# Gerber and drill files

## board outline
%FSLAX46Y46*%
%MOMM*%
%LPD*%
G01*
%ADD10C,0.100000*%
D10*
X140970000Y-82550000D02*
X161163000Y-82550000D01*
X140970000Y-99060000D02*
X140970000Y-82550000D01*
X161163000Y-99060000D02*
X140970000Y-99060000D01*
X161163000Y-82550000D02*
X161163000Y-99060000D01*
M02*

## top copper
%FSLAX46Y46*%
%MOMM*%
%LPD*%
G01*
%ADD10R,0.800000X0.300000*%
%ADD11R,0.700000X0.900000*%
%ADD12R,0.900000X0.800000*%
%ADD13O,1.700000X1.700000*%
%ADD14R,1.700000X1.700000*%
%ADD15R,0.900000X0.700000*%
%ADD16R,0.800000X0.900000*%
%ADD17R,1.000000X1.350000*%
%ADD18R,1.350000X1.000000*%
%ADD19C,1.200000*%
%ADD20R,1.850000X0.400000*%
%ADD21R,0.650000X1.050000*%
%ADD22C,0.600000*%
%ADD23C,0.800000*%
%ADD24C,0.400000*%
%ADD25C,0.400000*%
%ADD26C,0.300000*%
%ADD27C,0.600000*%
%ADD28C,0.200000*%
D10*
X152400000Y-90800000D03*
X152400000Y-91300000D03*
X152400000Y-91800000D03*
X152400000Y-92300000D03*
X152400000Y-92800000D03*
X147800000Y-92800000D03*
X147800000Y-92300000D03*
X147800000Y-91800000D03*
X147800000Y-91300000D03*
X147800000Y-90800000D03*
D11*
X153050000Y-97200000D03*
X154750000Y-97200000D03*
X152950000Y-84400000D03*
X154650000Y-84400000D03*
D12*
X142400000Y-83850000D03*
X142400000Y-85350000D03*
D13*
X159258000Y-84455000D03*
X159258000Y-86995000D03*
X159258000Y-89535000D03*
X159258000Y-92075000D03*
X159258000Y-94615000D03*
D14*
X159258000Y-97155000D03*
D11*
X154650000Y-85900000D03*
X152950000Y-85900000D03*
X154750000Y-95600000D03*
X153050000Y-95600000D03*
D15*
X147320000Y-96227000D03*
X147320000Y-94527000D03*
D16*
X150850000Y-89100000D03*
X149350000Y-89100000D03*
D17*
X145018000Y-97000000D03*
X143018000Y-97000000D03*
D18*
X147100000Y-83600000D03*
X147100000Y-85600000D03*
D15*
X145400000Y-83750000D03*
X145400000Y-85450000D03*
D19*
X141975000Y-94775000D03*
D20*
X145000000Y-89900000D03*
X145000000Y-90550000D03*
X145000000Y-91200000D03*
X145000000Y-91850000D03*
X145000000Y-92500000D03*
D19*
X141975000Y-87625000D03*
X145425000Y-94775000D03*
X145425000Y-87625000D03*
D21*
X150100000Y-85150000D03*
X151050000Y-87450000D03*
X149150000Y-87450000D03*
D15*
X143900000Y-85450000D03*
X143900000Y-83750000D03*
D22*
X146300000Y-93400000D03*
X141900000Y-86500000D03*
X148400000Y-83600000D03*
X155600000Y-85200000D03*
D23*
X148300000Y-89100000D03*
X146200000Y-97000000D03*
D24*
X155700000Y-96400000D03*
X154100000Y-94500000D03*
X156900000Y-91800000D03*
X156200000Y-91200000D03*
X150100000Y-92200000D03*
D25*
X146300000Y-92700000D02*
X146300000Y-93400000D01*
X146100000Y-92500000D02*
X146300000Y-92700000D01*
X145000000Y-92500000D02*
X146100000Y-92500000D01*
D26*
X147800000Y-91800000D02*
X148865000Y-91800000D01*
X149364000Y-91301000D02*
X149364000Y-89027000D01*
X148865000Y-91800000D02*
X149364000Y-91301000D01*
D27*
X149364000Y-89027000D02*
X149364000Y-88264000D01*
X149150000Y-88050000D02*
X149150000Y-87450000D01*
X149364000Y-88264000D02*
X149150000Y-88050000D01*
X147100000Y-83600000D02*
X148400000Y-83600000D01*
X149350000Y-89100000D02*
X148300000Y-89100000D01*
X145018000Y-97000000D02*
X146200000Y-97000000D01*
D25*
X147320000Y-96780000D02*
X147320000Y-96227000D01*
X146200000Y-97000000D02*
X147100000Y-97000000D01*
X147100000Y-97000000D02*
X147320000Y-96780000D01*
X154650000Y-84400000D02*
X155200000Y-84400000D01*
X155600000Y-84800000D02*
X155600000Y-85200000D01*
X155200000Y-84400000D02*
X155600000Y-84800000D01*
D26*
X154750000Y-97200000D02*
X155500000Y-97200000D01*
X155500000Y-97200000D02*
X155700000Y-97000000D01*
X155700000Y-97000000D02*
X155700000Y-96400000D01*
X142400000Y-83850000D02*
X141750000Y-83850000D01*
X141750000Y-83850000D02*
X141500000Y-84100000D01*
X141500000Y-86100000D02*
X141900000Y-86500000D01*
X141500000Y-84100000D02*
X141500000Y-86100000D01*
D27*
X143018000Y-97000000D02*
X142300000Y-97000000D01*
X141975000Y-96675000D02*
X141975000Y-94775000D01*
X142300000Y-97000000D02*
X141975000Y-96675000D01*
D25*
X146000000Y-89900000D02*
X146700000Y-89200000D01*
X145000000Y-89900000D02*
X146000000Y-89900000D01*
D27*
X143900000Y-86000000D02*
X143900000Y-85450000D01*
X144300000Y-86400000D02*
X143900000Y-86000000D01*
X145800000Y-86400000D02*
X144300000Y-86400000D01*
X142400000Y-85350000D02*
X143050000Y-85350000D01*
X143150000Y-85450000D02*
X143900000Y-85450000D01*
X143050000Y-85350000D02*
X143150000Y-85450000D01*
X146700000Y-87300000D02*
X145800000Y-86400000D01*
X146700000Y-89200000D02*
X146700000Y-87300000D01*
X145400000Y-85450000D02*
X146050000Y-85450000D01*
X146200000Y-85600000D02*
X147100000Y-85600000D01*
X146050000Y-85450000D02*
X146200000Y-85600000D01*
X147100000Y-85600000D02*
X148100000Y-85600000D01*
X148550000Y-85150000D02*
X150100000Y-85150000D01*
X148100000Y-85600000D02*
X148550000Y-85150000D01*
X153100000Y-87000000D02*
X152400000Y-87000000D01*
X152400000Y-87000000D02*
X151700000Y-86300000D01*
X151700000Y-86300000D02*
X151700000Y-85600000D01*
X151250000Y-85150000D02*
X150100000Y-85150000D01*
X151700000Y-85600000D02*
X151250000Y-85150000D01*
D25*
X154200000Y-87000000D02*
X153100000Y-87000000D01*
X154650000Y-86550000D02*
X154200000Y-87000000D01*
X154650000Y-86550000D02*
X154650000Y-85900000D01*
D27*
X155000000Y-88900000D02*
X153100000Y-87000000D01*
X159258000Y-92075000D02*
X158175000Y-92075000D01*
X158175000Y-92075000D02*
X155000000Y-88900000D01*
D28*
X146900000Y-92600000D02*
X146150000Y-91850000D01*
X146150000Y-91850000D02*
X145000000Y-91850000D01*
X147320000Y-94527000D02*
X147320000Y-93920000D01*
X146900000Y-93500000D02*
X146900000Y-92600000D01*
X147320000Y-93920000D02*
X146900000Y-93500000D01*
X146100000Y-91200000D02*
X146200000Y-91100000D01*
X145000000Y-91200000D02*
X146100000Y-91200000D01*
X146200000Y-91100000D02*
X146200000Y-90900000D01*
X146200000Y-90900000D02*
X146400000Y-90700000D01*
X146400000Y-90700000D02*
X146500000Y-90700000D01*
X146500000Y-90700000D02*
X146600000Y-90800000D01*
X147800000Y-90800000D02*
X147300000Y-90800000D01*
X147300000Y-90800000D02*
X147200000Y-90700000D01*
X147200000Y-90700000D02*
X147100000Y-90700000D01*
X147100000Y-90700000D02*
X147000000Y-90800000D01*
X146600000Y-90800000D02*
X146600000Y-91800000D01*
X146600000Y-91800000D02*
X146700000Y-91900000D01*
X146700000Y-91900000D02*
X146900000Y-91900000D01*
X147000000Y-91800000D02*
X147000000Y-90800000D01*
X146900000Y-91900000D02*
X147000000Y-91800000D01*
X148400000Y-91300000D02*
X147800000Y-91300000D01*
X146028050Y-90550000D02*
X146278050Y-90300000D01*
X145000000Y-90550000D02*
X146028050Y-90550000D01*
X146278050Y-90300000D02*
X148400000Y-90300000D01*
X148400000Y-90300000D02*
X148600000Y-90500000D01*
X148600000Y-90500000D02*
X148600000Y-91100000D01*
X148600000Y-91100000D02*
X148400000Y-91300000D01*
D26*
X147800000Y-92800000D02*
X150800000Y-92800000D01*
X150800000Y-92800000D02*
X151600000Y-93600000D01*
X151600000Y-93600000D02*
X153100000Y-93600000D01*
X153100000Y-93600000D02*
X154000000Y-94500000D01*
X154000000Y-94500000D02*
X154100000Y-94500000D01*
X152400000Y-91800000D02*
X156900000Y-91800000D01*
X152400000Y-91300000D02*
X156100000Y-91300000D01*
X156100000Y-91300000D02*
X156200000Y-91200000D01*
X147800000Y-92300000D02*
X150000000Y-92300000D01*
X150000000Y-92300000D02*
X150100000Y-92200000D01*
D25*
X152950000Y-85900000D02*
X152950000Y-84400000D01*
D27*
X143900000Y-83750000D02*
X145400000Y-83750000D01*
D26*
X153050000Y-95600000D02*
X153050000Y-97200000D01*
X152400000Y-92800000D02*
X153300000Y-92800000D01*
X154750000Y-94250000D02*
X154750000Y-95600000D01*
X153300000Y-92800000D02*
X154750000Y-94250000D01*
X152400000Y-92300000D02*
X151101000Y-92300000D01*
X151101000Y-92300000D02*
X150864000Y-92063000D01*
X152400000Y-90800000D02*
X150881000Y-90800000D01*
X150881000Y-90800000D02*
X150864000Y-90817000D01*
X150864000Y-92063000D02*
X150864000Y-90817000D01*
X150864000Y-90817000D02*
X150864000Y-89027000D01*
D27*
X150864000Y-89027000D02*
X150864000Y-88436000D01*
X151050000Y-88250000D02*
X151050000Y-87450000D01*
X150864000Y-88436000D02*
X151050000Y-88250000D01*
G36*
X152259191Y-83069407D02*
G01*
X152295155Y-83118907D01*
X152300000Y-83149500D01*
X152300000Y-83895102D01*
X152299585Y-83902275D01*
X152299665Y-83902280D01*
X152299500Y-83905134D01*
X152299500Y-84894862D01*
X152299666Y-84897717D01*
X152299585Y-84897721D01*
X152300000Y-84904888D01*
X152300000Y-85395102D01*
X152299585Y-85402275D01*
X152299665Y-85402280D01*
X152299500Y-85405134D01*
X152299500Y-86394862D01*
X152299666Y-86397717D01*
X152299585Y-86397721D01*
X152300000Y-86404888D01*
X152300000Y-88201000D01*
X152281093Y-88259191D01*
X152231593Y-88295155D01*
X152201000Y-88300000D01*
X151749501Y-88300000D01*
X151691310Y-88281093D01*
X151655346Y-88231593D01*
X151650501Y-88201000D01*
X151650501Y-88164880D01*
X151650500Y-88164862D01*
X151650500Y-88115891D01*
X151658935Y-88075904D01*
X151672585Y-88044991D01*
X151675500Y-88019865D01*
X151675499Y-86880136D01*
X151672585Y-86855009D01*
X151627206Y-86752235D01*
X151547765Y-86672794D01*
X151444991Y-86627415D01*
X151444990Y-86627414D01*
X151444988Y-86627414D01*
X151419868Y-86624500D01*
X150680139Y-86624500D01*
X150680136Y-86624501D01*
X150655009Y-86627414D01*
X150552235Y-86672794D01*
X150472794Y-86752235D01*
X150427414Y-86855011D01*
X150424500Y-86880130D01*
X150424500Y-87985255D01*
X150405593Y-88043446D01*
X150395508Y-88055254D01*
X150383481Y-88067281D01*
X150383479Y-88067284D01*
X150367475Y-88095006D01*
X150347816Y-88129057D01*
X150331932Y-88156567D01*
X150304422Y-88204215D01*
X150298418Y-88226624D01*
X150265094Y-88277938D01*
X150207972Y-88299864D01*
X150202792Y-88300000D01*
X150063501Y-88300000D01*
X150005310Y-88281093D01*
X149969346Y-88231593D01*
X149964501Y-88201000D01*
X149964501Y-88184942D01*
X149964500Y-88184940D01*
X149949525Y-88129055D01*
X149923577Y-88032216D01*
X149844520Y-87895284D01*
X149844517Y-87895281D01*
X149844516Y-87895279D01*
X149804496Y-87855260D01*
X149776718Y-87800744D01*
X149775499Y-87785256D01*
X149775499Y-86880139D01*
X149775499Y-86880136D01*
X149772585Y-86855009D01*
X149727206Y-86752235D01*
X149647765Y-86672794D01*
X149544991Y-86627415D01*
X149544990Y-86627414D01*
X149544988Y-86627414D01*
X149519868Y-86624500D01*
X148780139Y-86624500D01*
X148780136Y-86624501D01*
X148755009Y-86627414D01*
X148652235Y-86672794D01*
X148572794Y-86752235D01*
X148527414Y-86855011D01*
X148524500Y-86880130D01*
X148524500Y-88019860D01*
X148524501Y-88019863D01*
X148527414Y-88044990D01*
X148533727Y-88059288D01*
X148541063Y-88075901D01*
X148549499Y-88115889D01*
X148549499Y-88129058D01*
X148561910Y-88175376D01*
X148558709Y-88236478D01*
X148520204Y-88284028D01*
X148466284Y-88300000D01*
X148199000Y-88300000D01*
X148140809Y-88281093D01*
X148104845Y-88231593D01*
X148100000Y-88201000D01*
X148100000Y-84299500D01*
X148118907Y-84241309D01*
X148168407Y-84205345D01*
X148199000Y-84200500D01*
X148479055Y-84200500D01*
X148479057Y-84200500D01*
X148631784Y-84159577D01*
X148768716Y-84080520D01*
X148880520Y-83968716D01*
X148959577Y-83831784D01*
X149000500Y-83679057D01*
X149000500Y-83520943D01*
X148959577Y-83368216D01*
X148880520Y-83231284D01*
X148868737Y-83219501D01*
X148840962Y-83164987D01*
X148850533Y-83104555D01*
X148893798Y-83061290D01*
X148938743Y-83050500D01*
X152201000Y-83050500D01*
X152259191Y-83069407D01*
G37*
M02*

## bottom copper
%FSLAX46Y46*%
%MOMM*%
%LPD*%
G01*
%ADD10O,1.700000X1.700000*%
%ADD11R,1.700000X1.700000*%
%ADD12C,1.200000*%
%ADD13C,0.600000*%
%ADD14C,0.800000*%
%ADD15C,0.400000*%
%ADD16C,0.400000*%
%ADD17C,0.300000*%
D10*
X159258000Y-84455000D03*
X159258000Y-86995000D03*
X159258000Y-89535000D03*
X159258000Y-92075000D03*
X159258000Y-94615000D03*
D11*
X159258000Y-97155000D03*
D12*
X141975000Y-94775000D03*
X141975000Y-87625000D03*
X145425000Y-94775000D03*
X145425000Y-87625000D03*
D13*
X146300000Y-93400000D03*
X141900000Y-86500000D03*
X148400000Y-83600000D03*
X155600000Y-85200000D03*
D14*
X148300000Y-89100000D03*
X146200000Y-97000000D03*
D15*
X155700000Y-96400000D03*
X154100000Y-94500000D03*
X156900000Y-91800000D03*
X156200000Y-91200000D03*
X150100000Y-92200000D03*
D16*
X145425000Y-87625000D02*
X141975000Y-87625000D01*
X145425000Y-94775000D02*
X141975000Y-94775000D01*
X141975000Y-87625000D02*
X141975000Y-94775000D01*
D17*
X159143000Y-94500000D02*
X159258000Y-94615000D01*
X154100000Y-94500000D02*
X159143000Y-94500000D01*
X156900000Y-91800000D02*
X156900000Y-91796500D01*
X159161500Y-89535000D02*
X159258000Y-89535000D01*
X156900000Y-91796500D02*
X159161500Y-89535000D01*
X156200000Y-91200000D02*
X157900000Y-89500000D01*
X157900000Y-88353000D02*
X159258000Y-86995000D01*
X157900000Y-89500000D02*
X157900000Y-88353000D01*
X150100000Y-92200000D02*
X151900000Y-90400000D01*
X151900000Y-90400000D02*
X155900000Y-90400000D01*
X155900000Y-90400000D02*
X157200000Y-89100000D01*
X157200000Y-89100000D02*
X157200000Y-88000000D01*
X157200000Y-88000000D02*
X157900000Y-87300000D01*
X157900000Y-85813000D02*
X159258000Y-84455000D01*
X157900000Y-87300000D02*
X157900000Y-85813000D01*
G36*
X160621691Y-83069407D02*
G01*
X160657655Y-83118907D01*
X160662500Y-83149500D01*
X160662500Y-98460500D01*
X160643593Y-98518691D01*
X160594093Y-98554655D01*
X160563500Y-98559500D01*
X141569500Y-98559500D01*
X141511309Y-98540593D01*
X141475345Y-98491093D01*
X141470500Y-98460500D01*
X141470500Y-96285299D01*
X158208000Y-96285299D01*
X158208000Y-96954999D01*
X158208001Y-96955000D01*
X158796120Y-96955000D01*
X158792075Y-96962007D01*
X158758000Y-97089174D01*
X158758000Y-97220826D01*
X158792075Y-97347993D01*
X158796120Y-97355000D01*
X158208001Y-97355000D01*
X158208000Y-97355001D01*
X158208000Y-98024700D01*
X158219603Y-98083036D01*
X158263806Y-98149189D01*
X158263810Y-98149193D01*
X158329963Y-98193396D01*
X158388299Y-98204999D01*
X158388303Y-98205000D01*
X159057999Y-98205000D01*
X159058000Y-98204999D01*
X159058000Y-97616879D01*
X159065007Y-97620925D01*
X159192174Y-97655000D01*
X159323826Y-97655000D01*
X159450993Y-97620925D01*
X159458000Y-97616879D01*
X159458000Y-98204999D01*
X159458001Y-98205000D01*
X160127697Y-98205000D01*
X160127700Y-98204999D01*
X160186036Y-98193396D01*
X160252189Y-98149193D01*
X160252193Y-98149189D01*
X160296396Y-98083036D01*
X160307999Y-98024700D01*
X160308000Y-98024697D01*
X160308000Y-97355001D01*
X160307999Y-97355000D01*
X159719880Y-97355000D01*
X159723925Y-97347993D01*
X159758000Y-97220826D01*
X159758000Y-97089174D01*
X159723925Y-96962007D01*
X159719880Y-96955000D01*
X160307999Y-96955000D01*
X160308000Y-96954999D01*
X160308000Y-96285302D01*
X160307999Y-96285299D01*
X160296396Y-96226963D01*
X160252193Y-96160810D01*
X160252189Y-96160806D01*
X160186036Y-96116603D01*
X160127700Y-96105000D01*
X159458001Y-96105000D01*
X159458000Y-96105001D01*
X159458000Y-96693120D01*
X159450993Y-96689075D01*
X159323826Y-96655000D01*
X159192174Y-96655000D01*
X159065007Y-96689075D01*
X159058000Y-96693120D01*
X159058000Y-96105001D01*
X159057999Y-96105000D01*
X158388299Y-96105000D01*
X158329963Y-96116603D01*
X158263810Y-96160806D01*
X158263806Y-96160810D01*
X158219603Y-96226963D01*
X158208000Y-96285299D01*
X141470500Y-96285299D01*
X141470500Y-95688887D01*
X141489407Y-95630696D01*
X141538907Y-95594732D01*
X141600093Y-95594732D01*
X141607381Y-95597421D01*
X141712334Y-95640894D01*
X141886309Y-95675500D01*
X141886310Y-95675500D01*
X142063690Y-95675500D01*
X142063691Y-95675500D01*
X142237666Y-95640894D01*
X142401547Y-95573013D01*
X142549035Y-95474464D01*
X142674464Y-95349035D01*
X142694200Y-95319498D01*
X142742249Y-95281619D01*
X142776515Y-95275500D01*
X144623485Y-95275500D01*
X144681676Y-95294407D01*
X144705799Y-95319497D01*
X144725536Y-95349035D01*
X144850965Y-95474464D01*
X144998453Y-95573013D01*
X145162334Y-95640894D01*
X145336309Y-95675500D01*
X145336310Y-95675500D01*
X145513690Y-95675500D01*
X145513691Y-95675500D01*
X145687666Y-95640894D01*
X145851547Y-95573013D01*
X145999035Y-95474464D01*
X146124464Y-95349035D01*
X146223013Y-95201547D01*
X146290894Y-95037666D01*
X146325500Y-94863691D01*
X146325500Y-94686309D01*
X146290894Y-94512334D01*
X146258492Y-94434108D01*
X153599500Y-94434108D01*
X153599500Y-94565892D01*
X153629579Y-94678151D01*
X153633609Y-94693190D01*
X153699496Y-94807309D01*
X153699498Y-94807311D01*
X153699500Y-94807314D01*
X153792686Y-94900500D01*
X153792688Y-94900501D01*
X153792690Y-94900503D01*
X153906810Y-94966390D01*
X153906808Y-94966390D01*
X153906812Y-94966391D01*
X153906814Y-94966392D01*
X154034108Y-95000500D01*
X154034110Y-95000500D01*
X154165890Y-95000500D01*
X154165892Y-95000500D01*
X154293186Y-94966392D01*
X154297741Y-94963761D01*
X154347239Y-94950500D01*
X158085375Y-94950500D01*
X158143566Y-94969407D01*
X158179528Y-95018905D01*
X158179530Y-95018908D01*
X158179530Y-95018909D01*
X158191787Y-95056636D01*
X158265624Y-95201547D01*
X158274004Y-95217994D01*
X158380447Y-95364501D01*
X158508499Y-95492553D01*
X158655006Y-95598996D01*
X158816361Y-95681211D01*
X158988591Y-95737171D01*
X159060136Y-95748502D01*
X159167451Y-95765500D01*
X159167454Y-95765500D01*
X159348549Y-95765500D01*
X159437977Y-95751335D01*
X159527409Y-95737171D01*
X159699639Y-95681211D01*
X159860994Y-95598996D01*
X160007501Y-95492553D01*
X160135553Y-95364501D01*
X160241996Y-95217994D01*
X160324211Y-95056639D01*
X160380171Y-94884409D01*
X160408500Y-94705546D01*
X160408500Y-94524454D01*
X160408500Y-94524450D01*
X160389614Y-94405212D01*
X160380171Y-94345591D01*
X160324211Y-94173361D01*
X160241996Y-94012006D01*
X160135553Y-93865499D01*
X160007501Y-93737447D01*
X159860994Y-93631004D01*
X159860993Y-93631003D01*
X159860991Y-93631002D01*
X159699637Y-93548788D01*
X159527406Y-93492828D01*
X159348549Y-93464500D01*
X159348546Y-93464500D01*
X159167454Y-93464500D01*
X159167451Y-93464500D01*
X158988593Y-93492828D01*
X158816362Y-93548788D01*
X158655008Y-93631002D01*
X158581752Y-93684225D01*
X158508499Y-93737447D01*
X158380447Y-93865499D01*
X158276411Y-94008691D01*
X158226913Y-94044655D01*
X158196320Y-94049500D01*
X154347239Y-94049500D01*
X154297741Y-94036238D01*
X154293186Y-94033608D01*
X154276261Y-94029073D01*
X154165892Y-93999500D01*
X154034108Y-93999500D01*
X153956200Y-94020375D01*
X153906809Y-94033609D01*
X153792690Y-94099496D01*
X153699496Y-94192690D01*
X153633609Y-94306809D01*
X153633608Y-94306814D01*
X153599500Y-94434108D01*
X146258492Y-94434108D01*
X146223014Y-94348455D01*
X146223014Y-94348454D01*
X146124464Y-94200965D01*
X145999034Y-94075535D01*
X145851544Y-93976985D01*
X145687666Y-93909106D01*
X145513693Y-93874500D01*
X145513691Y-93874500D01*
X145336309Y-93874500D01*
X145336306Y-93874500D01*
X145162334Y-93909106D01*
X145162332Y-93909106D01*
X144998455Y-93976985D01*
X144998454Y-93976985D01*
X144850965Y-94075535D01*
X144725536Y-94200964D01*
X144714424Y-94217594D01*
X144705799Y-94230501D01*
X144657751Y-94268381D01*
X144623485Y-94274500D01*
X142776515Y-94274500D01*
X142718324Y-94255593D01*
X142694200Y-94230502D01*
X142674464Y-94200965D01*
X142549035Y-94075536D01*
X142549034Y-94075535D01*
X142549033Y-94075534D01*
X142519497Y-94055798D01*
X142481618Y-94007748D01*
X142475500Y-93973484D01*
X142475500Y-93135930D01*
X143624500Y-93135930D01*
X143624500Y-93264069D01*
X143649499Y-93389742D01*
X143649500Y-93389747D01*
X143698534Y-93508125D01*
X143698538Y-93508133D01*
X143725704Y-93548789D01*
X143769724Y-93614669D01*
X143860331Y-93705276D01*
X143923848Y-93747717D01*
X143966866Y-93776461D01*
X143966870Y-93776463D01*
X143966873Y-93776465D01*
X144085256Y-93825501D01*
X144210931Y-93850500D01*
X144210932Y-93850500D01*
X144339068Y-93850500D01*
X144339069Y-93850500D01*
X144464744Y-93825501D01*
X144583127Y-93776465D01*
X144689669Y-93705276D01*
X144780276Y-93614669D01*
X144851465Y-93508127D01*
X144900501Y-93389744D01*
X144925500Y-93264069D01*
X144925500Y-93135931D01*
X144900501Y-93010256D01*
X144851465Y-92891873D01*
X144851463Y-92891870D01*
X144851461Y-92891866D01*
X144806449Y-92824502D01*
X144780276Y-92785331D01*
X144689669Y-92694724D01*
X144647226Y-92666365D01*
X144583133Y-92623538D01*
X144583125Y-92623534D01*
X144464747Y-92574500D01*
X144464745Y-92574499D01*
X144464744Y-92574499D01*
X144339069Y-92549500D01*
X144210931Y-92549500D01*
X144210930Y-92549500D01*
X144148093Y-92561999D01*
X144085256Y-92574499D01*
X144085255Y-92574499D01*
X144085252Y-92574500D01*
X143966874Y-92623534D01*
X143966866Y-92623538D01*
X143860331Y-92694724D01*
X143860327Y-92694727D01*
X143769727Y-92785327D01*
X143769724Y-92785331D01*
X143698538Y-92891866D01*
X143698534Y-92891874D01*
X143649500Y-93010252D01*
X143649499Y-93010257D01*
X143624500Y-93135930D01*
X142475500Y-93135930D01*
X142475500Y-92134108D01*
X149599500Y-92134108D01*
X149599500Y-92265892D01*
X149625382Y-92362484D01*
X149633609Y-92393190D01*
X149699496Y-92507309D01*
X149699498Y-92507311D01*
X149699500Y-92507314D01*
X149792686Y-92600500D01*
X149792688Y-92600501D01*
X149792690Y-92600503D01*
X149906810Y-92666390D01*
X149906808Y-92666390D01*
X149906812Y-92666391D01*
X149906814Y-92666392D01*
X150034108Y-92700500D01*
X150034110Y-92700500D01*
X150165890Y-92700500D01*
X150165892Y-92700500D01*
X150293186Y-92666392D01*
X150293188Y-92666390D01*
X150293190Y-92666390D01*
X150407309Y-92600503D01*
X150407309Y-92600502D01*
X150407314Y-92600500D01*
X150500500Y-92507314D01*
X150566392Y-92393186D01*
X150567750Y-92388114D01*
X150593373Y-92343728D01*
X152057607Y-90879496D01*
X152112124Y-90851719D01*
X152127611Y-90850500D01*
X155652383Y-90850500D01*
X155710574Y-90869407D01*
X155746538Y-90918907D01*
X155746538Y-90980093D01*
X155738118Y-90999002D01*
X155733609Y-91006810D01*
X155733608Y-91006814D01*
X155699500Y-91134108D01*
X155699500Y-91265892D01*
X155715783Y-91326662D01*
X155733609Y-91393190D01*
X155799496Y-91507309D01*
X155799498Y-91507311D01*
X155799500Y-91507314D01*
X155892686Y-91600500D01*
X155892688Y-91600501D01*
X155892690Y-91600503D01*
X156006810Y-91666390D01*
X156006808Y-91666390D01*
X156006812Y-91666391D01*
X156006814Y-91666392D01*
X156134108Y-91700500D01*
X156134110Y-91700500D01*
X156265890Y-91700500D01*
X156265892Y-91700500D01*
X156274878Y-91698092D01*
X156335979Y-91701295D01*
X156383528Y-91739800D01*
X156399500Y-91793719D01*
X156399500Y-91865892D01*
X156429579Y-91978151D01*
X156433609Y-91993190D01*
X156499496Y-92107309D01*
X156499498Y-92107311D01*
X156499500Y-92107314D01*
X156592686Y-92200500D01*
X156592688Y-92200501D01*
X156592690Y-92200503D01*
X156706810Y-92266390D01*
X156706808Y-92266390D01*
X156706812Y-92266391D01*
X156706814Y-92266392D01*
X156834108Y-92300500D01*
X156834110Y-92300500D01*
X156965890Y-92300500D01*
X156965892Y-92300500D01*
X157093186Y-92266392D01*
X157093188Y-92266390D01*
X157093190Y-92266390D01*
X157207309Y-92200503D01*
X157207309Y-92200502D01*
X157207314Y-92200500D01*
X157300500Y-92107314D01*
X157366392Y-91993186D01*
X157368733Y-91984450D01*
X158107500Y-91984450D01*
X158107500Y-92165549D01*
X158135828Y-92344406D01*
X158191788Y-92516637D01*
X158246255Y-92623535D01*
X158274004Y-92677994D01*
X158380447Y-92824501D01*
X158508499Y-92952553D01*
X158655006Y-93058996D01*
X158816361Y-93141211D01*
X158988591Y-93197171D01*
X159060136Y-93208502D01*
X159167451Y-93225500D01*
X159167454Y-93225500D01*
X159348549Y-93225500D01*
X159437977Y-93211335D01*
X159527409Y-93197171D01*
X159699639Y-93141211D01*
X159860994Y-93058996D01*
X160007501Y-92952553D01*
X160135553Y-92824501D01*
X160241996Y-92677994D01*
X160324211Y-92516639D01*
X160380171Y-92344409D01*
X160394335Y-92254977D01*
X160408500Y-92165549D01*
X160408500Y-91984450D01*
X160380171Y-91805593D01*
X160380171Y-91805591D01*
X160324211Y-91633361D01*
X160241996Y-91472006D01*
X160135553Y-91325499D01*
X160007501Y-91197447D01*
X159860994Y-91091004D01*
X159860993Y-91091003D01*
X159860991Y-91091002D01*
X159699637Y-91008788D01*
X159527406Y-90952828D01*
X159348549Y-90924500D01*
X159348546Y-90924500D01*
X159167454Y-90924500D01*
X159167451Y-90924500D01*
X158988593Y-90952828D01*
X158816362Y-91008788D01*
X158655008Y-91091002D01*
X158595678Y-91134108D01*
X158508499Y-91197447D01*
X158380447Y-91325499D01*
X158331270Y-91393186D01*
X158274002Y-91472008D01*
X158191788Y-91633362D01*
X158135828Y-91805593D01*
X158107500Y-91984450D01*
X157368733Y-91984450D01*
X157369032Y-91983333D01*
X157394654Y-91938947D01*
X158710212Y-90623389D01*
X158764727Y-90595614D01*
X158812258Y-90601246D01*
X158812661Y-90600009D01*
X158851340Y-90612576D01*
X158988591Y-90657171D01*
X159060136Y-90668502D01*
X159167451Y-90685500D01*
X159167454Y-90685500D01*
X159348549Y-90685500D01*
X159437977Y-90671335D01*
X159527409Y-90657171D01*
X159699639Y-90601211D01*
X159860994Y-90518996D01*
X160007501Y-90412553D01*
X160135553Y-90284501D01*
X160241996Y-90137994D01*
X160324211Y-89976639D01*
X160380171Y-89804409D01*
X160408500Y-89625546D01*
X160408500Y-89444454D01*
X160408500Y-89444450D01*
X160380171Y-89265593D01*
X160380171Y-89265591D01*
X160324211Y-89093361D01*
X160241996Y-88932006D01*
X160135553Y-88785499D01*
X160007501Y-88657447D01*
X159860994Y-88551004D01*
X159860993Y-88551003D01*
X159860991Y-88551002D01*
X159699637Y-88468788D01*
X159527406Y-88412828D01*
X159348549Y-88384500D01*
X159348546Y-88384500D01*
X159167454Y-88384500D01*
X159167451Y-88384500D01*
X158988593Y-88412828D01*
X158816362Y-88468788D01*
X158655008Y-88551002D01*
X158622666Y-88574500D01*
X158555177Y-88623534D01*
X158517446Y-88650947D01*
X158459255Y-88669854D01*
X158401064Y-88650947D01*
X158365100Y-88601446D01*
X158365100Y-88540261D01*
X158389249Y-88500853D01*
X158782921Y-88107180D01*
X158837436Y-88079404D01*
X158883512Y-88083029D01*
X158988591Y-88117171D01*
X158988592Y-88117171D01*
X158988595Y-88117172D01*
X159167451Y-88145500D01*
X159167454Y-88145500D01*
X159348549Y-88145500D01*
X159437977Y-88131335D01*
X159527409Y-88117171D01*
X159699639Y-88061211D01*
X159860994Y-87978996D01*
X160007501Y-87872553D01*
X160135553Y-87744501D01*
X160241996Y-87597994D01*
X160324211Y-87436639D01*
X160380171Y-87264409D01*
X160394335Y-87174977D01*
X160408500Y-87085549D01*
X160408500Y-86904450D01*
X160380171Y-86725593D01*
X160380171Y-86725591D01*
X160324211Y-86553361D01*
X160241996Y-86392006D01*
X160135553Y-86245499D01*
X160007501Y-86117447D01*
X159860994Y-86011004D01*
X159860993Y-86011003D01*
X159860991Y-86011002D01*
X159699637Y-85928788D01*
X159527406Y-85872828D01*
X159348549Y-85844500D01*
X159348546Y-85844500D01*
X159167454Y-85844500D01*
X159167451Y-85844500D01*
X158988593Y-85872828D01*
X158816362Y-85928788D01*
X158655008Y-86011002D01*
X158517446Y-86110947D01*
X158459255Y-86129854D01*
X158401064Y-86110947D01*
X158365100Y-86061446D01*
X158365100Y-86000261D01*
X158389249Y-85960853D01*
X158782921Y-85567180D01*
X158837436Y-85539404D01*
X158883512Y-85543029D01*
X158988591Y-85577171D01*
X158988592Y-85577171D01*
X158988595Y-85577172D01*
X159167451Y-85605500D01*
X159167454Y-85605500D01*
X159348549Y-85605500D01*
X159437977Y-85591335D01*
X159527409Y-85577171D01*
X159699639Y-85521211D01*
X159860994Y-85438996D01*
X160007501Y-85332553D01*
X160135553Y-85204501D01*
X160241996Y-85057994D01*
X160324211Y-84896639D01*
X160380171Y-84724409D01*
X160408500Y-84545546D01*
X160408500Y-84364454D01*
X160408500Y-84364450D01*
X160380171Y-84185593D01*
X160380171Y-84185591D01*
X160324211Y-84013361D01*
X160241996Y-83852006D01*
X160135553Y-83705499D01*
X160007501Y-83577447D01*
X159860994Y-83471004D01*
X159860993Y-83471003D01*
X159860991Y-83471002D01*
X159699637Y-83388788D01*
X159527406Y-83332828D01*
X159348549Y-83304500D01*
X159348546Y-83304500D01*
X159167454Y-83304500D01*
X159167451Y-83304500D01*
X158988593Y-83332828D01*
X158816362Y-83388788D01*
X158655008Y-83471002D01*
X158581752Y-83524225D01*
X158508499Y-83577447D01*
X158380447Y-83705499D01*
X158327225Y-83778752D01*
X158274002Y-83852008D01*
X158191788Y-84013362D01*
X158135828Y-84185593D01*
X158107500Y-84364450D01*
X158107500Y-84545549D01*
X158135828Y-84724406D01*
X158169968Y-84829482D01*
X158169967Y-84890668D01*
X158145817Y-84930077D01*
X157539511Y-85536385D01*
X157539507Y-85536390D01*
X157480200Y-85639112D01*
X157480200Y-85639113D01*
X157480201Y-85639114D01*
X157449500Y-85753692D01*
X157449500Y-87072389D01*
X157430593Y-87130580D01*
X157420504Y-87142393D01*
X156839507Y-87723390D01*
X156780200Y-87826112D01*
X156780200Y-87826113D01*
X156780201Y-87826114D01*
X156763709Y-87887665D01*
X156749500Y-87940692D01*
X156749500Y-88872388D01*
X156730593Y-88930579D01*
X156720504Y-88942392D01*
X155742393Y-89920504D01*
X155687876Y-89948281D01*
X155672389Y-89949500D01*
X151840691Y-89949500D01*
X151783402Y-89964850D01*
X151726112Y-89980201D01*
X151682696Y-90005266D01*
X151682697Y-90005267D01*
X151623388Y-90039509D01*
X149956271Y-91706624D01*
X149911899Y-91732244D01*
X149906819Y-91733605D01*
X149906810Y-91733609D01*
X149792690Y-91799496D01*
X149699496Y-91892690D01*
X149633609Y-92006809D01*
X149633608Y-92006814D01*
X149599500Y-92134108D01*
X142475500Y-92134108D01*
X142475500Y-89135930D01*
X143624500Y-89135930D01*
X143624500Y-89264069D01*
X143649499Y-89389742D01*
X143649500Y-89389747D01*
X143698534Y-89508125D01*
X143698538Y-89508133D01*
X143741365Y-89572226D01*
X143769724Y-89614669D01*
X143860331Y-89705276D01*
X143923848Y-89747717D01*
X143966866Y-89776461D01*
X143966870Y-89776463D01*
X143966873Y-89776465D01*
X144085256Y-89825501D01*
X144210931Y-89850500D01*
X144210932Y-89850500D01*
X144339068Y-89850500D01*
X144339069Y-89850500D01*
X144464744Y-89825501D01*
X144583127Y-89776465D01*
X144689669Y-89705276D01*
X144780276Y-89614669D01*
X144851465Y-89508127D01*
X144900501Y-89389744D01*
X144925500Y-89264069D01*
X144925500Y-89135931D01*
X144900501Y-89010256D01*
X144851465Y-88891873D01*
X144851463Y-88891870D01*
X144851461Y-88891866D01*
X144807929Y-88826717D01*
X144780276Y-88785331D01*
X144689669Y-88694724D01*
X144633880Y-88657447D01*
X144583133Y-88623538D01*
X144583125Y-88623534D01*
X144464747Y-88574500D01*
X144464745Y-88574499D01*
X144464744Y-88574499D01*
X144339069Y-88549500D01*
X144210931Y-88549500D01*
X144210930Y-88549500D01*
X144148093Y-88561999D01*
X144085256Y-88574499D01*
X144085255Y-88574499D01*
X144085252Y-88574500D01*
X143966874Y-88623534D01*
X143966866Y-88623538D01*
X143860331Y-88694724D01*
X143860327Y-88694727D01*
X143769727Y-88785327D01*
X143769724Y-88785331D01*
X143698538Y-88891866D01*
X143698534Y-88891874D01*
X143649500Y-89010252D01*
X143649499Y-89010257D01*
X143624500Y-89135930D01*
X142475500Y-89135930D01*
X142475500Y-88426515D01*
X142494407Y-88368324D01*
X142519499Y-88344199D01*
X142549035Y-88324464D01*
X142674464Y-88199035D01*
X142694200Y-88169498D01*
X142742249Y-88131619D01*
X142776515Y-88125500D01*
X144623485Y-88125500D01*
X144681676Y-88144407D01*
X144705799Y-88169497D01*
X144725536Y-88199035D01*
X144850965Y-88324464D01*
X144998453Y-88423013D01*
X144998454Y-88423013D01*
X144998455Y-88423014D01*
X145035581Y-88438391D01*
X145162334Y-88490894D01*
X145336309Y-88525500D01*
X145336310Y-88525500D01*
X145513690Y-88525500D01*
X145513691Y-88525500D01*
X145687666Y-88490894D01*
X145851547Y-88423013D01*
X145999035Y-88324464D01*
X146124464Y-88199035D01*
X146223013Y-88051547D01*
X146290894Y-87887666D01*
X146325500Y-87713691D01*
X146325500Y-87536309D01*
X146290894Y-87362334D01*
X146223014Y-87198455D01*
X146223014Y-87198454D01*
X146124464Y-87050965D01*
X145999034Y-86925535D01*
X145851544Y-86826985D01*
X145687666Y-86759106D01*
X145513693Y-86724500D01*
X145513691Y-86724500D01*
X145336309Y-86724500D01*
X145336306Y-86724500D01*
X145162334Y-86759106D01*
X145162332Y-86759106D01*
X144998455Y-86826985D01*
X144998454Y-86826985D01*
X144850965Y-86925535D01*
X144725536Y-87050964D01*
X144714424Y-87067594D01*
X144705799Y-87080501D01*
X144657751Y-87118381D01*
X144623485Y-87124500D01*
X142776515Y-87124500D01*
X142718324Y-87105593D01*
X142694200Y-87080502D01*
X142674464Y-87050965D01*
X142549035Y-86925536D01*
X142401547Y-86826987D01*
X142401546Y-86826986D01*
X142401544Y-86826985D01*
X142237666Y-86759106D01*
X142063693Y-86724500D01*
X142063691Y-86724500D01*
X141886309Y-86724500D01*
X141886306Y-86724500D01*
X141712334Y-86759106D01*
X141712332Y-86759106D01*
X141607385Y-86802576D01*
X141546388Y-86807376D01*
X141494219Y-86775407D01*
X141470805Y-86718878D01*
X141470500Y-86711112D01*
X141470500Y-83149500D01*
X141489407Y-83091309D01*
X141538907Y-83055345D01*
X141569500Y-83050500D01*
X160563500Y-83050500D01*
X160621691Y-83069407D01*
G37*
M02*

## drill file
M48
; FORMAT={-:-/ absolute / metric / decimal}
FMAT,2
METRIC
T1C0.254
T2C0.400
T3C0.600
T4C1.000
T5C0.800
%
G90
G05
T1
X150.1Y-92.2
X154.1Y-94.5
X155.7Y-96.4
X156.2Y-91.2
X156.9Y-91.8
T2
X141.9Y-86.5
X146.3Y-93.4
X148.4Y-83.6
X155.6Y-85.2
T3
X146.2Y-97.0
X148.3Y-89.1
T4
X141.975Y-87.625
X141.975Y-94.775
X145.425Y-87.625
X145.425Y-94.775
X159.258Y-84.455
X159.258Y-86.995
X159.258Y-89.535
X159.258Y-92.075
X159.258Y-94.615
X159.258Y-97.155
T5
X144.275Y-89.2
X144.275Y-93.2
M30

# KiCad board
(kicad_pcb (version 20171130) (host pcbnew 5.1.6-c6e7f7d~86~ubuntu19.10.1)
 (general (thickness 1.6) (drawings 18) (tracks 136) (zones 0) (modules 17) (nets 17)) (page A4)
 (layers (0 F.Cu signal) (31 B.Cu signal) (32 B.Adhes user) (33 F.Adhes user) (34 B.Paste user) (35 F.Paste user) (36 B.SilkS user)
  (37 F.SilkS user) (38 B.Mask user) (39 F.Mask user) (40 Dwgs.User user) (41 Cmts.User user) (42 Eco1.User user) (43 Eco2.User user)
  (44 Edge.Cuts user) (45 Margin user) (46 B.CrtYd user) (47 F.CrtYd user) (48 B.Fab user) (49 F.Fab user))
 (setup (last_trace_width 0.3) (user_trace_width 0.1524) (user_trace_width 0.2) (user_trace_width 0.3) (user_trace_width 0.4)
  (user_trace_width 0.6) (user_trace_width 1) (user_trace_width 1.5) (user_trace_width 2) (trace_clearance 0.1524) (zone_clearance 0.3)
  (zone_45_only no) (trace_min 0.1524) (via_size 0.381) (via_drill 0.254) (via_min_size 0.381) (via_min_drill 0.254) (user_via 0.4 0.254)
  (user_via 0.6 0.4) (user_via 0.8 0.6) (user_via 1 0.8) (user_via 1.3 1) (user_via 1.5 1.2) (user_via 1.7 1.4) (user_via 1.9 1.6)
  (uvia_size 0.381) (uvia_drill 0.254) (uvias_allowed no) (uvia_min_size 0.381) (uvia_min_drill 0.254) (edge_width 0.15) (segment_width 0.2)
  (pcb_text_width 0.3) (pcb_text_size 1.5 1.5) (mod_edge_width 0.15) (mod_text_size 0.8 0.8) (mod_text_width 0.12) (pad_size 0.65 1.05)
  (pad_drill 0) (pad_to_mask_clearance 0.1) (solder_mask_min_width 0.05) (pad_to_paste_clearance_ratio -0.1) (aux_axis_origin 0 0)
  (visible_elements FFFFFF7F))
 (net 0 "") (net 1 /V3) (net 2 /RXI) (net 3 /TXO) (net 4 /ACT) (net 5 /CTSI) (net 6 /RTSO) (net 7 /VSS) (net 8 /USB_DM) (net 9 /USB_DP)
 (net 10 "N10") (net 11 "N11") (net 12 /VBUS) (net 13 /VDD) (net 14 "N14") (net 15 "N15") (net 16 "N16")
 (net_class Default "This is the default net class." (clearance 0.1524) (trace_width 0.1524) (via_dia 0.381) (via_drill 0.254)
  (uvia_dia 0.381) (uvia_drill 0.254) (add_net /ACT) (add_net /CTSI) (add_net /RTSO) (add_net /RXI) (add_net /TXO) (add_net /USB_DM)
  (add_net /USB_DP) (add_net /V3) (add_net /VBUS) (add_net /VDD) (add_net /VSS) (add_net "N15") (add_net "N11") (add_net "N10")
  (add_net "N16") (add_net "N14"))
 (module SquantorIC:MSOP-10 (layer F.Cu) (at 150.1 91.8)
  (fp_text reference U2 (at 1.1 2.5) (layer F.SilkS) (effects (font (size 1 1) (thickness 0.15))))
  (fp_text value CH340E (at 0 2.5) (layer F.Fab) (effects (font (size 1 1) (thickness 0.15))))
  (pad 10 smd rect (at 2.3 -1) (size 0.8 0.3) (layers F.Cu F.Paste F.Mask) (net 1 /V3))
  (pad 9 smd rect (at 2.3 -0.5) (size 0.8 0.3) (layers F.Cu F.Paste F.Mask) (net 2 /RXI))
  (pad 8 smd rect (at 2.3 0) (size 0.8 0.3) (layers F.Cu F.Paste F.Mask) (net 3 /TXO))
  (pad 7 smd rect (at 2.3 0.5) (size 0.8 0.3) (layers F.Cu F.Paste F.Mask) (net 1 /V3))
  (pad 6 smd rect (at 2.3 1) (size 0.8 0.3) (layers F.Cu F.Paste F.Mask) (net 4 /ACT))
  (pad 5 smd rect (at -2.3 1) (size 0.8 0.3) (layers F.Cu F.Paste F.Mask) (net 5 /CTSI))
  (pad 4 smd rect (at -2.3 0.5) (size 0.8 0.3) (layers F.Cu F.Paste F.Mask) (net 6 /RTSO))
  (pad 3 smd rect (at -2.3 0) (size 0.8 0.3) (layers F.Cu F.Paste F.Mask) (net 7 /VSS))
  (pad 2 smd rect (at -2.3 -0.5) (size 0.8 0.3) (layers F.Cu F.Paste F.Mask) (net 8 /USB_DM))
  (pad 1 smd rect (at -2.3 -1) (size 0.8 0.3) (layers F.Cu F.Paste F.Mask) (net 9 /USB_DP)))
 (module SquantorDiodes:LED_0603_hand (layer F.Cu) (at 153.9 97.2 180)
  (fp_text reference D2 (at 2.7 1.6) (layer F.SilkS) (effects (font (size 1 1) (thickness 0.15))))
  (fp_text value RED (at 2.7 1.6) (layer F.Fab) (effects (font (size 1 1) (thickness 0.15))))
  (pad 2 smd rect (at 0.85 0 180) (size 0.7 0.9) (layers F.Cu F.Paste F.Mask) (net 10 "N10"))
  (pad 1 smd rect (at -0.85 0 180) (size 0.7 0.9) (layers F.Cu F.Paste F.Mask) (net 7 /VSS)))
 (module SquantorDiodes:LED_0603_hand (layer F.Cu) (at 153.8 84.4 180)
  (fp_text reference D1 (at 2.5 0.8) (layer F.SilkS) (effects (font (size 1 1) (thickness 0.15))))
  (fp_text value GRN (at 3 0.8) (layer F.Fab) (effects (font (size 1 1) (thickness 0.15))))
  (pad 2 smd rect (at 0.85 0 180) (size 0.7 0.9) (layers F.Cu F.Paste F.Mask) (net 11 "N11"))
  (pad 1 smd rect (at -0.85 0 180) (size 0.7 0.9) (layers F.Cu F.Paste F.Mask) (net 7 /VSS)))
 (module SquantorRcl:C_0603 (layer F.Cu) (at 142.4 84.6 90)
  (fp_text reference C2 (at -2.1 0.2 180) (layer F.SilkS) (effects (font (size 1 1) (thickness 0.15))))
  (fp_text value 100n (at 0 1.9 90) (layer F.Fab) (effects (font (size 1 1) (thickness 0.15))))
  (pad 2 smd rect (at 0.75 0 90) (size 0.8 0.9) (layers F.Cu F.Paste F.Mask) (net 7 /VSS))
  (pad 1 smd rect (at -0.75 0 90) (size 0.8 0.9) (layers F.Cu F.Paste F.Mask) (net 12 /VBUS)))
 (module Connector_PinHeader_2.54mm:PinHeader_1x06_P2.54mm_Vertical (layer F.Cu) (at 159.258 97.155 180)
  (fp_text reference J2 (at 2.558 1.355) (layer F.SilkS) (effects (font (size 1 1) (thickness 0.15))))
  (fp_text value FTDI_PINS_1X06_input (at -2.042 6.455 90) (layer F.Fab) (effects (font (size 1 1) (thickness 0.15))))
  (pad 6 thru_hole oval (at 0 12.7 180) (size 1.7 1.7) (drill 1) (layers *.Cu *.Mask) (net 6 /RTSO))
  (pad 5 thru_hole oval (at 0 10.16 180) (size 1.7 1.7) (drill 1) (layers *.Cu *.Mask) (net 2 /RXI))
  (pad 4 thru_hole oval (at 0 7.62 180) (size 1.7 1.7) (drill 1) (layers *.Cu *.Mask) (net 3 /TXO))
  (pad 3 thru_hole oval (at 0 5.08 180) (size 1.7 1.7) (drill 1) (layers *.Cu *.Mask) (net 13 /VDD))
  (pad 2 thru_hole oval (at 0 2.54 180) (size 1.7 1.7) (drill 1) (layers *.Cu *.Mask) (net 5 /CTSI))
  (pad 1 thru_hole rect (at 0 0 180) (size 1.7 1.7) (drill 1) (layers *.Cu *.Mask) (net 7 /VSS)))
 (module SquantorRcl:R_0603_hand (layer F.Cu) (at 153.8 85.9)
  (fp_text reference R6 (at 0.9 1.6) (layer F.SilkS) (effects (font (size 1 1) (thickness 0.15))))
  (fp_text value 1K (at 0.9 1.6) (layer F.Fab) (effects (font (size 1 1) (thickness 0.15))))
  (pad 2 smd rect (at 0.85 0) (size 0.7 0.9) (layers F.Cu F.Paste F.Mask) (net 13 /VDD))
  (pad 1 smd rect (at -0.85 0) (size 0.7 0.9) (layers F.Cu F.Paste F.Mask) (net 11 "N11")))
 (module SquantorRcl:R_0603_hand (layer F.Cu) (at 153.9 95.6)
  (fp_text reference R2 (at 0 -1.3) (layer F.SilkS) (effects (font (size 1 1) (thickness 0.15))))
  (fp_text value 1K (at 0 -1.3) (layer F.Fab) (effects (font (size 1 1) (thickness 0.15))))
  (pad 2 smd rect (at 0.85 0) (size 0.7 0.9) (layers F.Cu F.Paste F.Mask) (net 4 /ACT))
  (pad 1 smd rect (at -0.85 0) (size 0.7 0.9) (layers F.Cu F.Paste F.Mask) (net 10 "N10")))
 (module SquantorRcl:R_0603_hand (layer F.Cu) (at 147.32 95.377 270)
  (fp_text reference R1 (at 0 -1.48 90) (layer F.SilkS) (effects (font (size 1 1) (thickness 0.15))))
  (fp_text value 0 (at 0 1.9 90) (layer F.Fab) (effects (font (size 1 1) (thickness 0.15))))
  (pad 2 smd rect (at 0.85 0 270) (size 0.7 0.9) (layers F.Cu F.Paste F.Mask) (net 7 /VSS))
  (pad 1 smd rect (at -0.85 0 270) (size 0.7 0.9) (layers F.Cu F.Paste F.Mask) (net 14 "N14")))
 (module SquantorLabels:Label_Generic (layer B.Cu) (at 151.4 95.6 180)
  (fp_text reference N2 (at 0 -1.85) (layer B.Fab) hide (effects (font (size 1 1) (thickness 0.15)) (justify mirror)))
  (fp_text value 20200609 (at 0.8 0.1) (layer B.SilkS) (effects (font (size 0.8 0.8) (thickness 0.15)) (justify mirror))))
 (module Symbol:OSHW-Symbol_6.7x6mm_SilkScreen (layer B.Cu) (at 150.6 91.8 180)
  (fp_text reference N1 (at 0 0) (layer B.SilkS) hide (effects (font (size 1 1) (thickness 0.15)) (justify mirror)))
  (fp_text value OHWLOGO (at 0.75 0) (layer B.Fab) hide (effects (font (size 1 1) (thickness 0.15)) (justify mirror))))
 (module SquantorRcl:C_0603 (layer F.Cu) (at 150.1 89.1)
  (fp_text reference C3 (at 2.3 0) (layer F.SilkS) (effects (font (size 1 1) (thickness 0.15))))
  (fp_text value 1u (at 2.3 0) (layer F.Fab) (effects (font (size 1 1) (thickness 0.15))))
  (pad 2 smd rect (at 0.75 0) (size 0.8 0.9) (layers F.Cu F.Paste F.Mask) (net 1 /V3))
  (pad 1 smd rect (at -0.75 0) (size 0.8 0.9) (layers F.Cu F.Paste F.Mask) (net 7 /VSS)))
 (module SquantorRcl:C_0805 (layer F.Cu) (at 144.018 97)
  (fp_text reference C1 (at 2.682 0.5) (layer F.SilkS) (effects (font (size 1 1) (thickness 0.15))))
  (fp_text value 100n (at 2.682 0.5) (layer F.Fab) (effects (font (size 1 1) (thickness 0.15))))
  (pad 2 smd rect (at 1 0) (size 1 1.35) (layers F.Cu F.Paste F.Mask) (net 7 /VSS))
  (pad 1 smd rect (at -1 0) (size 1 1.35) (layers F.Cu F.Paste F.Mask) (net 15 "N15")))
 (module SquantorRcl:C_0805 (layer F.Cu) (at 147.1 84.6 90)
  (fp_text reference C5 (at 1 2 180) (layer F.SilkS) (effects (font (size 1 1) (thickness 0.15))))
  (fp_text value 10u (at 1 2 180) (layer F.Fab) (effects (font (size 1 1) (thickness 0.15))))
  (pad 2 smd rect (at 1 0 90) (size 1 1.35) (layers F.Cu F.Paste F.Mask) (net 7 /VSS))
  (pad 1 smd rect (at -1 0 90) (size 1 1.35) (layers F.Cu F.Paste F.Mask) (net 13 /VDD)))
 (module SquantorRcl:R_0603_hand (layer F.Cu) (at 145.4 84.6 90)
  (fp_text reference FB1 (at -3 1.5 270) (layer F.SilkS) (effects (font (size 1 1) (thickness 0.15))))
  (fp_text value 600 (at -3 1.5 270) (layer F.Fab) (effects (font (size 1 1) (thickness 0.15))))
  (pad 2 smd rect (at 0.85 0 90) (size 0.7 0.9) (layers F.Cu F.Paste F.Mask) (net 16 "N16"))
  (pad 1 smd rect (at -0.85 0 90) (size 0.7 0.9) (layers F.Cu F.Paste F.Mask) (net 13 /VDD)))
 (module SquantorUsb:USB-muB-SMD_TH (layer F.Cu) (at 143.7 91.2 270)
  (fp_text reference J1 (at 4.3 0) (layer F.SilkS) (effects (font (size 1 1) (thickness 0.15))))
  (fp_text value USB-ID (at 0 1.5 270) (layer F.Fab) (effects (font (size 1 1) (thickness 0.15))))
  (pad S thru_hole circle (at 3.575 1.725 270) (size 1.2 1.2) (drill 1) (layers *.Cu *.Mask) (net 15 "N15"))
  (pad "" np_thru_hole circle (at 2 -0.575 270) (size 0.8 0.8) (drill 0.8) (layers *.Cu))
  (pad 1 smd rect (at -1.3 -1.3 270) (size 0.4 1.85) (layers F.Cu F.Paste F.Mask) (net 12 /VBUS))
  (pad 2 smd rect (at -0.65 -1.3 270) (size 0.4 1.85) (layers F.Cu F.Paste F.Mask) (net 8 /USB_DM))
  (pad 3 smd rect (at 0 -1.3 270) (size 0.4 1.85) (layers F.Cu F.Paste F.Mask) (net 9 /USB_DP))
  (pad 4 smd rect (at 0.65 -1.3 270) (size 0.4 1.85) (layers F.Cu F.Paste F.Mask) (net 14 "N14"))
  (pad 5 smd rect (at 1.3 -1.3 270) (size 0.4 1.85) (layers F.Cu F.Paste F.Mask) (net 7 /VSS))
  (pad "" np_thru_hole circle (at -2 -0.575 270) (size 0.8 0.8) (drill 0.8) (layers *.Cu))
  (pad S thru_hole circle (at -3.575 1.725 270) (size 1.2 1.2) (drill 1) (layers *.Cu *.Mask) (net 15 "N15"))
  (pad S thru_hole circle (at 3.575 -1.725 270) (size 1.2 1.2) (drill 1) (layers *.Cu *.Mask) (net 15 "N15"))
  (pad S thru_hole circle (at -3.575 -1.725 270) (size 1.2 1.2) (drill 1) (layers *.Cu *.Mask) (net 15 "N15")))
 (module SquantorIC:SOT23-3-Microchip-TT (layer F.Cu) (at 150.1 86.3)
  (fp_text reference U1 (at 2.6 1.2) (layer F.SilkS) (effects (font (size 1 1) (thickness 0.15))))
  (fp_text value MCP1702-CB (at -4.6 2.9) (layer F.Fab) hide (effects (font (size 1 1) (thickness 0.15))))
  (pad 3 smd rect (at 0 -1.15) (size 0.65 1.05) (layers F.Cu F.Paste F.Mask) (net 13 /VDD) (zone_connect 2))
  (pad 2 smd rect (at 0.95 1.15) (size 0.65 1.05) (layers F.Cu F.Paste F.Mask) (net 1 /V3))
  (pad 1 smd rect (at -0.95 1.15) (size 0.65 1.05) (layers F.Cu F.Paste F.Mask) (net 7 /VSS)))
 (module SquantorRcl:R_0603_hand (layer F.Cu) (at 143.9 84.6 270)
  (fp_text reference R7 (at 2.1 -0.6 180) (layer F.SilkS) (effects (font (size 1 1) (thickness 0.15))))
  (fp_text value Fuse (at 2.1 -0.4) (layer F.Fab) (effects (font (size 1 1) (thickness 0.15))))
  (pad 2 smd rect (at 0.85 0 270) (size 0.7 0.9) (layers F.Cu F.Paste F.Mask) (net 12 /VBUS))
  (pad 1 smd rect (at -0.85 0 270) (size 0.7 0.9) (layers F.Cu F.Paste F.Mask) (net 16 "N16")))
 (gr_line (start 140.97 82.55) (end 161.163 82.55) (layer Edge.Cuts) (width 0.1))
 (gr_line (start 140.97 99.06) (end 140.97 82.55) (layer Edge.Cuts) (width 0.1))
 (gr_line (start 161.163 99.06) (end 140.97 99.06) (layer Edge.Cuts) (width 0.1))
 (gr_line (start 161.163 82.55) (end 161.163 99.06) (layer Edge.Cuts) (width 0.1))
 (segment (start 146.3 92.7) (end 146.3 93.4) (width 0.4) (layer F.Cu) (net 7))
 (segment (start 146.1 92.5) (end 146.3 92.7) (width 0.4) (layer F.Cu) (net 7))
 (segment (start 145 92.5) (end 146.1 92.5) (width 0.4) (layer F.Cu) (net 7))
 (via (at 146.3 93.4) (size 0.6) (drill 0.4) (layers F.Cu B.Cu) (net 7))
 (segment (start 147.8 91.8) (end 148.865 91.8) (width 0.3) (layer F.Cu) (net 7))
 (segment (start 149.364 91.301) (end 149.364 89.027) (width 0.3) (layer F.Cu) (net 7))
 (segment (start 148.865 91.8) (end 149.364 91.301) (width 0.3) (layer F.Cu) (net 7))
 (segment (start 149.364 89.027) (end 149.364 88.264) (width 0.6) (layer F.Cu) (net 7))
 (segment (start 149.15 88.05) (end 149.15 87.45) (width 0.6) (layer F.Cu) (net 7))
 (segment (start 149.364 88.264) (end 149.15 88.05) (width 0.6) (layer F.Cu) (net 7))
 (via (at 141.9 86.5) (size 0.6) (drill 0.4) (layers F.Cu B.Cu) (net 7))
 (via (at 148.4 83.6) (size 0.6) (drill 0.4) (layers F.Cu B.Cu) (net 7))
 (segment (start 147.1 83.6) (end 148.4 83.6) (width 0.6) (layer F.Cu) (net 7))
 (via (at 155.6 85.2) (size 0.6) (drill 0.4) (layers F.Cu B.Cu) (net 7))
 (via (at 148.3 89.1) (size 0.8) (drill 0.6) (layers F.Cu B.Cu) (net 7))
 (segment (start 149.35 89.1) (end 148.3 89.1) (width 0.6) (layer F.Cu) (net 7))
 (via (at 146.2 97) (size 0.8) (drill 0.6) (layers F.Cu B.Cu) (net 7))
 (segment (start 145.018 97) (end 146.2 97) (width 0.6) (layer F.Cu) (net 7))
 (segment (start 147.32 96.78) (end 147.32 96.227) (width 0.4) (layer F.Cu) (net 7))
 (segment (start 146.2 97) (end 147.1 97) (width 0.4) (layer F.Cu) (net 7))
 (segment (start 147.1 97) (end 147.32 96.78) (width 0.4) (layer F.Cu) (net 7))
 (segment (start 154.65 84.4) (end 155.2 84.4) (width 0.4) (layer F.Cu) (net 7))
 (segment (start 155.6 84.8) (end 155.6 85.2) (width 0.4) (layer F.Cu) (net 7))
 (segment (start 155.2 84.4) (end 155.6 84.8) (width 0.4) (layer F.Cu) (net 7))
 (segment (start 154.75 97.2) (end 155.5 97.2) (width 0.3) (layer F.Cu) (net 7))
 (via (at 155.7 96.4) (size 0.4) (drill 0.254) (layers F.Cu B.Cu) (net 7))
 (segment (start 155.5 97.2) (end 155.7 97) (width 0.3) (layer F.Cu) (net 7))
 (segment (start 155.7 97) (end 155.7 96.4) (width 0.3) (layer F.Cu) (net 7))
 (segment (start 142.4 83.85) (end 141.75 83.85) (width 0.3) (layer F.Cu) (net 7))
 (segment (start 141.75 83.85) (end 141.5 84.1) (width 0.3) (layer F.Cu) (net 7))
 (segment (start 141.5 86.1) (end 141.9 86.5) (width 0.3) (layer F.Cu) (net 7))
 (segment (start 141.5 84.1) (end 141.5 86.1) (width 0.3) (layer F.Cu) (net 7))
 (segment (start 145.425 87.625) (end 141.975 87.625) (width 0.4) (layer B.Cu) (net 15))
 (segment (start 145.425 94.775) (end 141.975 94.775) (width 0.4) (layer B.Cu) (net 15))
 (segment (start 141.975 87.625) (end 141.975 94.775) (width 0.4) (layer B.Cu) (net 15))
 (segment (start 143.018 97) (end 142.3 97) (width 0.6) (layer F.Cu) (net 15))
 (segment (start 141.975 96.675) (end 141.975 94.775) (width 0.6) (layer F.Cu) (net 15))
 (segment (start 142.3 97) (end 141.975 96.675) (width 0.6) (layer F.Cu) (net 15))
 (segment (start 146 89.9) (end 146.7 89.2) (width 0.4) (layer F.Cu) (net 12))
 (segment (start 145 89.9) (end 146 89.9) (width 0.4) (layer F.Cu) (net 12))
 (segment (start 143.9 86) (end 143.9 85.45) (width 0.6) (layer F.Cu) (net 12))
 (segment (start 144.3 86.4) (end 143.9 86) (width 0.6) (layer F.Cu) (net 12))
 (segment (start 145.8 86.4) (end 144.3 86.4) (width 0.6) (layer F.Cu) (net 12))
 (segment (start 142.4 85.35) (end 143.05 85.35) (width 0.6) (layer F.Cu) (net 12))
 (segment (start 143.15 85.45) (end 143.9 85.45) (width 0.6) (layer F.Cu) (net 12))
 (segment (start 143.05 85.35) (end 143.15 85.45) (width 0.6) (layer F.Cu) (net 12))
 (segment (start 146.7 87.3) (end 145.8 86.4) (width 0.6) (layer F.Cu) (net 12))
 (segment (start 146.7 89.2) (end 146.7 87.3) (width 0.6) (layer F.Cu) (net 12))
 (segment (start 145.4 85.45) (end 146.05 85.45) (width 0.6) (layer F.Cu) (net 13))
 (segment (start 146.2 85.6) (end 147.1 85.6) (width 0.6) (layer F.Cu) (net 13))
 (segment (start 146.05 85.45) (end 146.2 85.6) (width 0.6) (layer F.Cu) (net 13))
 (segment (start 147.1 85.6) (end 148.1 85.6) (width 0.6) (layer F.Cu) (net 13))
 (segment (start 148.55 85.15) (end 150.1 85.15) (width 0.6) (layer F.Cu) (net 13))
 (segment (start 148.1 85.6) (end 148.55 85.15) (width 0.6) (layer F.Cu) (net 13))
 (segment (start 153.1 87) (end 152.4 87) (width 0.6) (layer F.Cu) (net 13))
 (segment (start 152.4 87) (end 151.7 86.3) (width 0.6) (layer F.Cu) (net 13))
 (segment (start 151.7 86.3) (end 151.7 85.6) (width 0.6) (layer F.Cu) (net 13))
 (segment (start 151.25 85.15) (end 150.1 85.15) (width 0.6) (layer F.Cu) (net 13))
 (segment (start 151.7 85.6) (end 151.25 85.15) (width 0.6) (layer F.Cu) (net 13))
 (segment (start 154.2 87) (end 153.1 87) (width 0.4) (layer F.Cu) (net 13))
 (segment (start 154.65 86.55) (end 154.2 87) (width 0.4) (layer F.Cu) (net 13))
 (segment (start 154.65 86.55) (end 154.65 85.9) (width 0.4) (layer F.Cu) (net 13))
 (segment (start 155 88.9) (end 153.1 87) (width 0.6) (layer F.Cu) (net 13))
 (segment (start 159.258 92.075) (end 158.175 92.075) (width 0.6) (layer F.Cu) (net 13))
 (segment (start 158.175 92.075) (end 155 88.9) (width 0.6) (layer F.Cu) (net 13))
 (segment (start 146.9 92.6) (end 146.15 91.85) (width 0.2) (layer F.Cu) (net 14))
 (segment (start 146.15 91.85) (end 145 91.85) (width 0.2) (layer F.Cu) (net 14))
 (segment (start 147.32 94.527) (end 147.32 93.92) (width 0.2) (layer F.Cu) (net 14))
 (segment (start 146.9 93.5) (end 146.9 92.6) (width 0.2) (layer F.Cu) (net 14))
 (segment (start 147.32 93.92) (end 146.9 93.5) (width 0.2) (layer F.Cu) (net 14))
 (segment (start 146.1 91.2) (end 146.2 91.1) (width 0.2) (layer F.Cu) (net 9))
 (segment (start 145 91.2) (end 146.1 91.2) (width 0.2) (layer F.Cu) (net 9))
 (segment (start 146.2 91.1) (end 146.2 90.9) (width 0.2) (layer F.Cu) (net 9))
 (segment (start 146.2 90.9) (end 146.4 90.7) (width 0.2) (layer F.Cu) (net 9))
 (segment (start 146.4 90.7) (end 146.5 90.7) (width 0.2) (layer F.Cu) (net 9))
 (segment (start 146.5 90.7) (end 146.6 90.8) (width 0.2) (layer F.Cu) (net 9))
 (segment (start 147.8 90.8) (end 147.3 90.8) (width 0.2) (layer F.Cu) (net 9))
 (segment (start 147.3 90.8) (end 147.2 90.7) (width 0.2) (layer F.Cu) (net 9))
 (segment (start 147.2 90.7) (end 147.1 90.7) (width 0.2) (layer F.Cu) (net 9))
 (segment (start 147.1 90.7) (end 147 90.8) (width 0.2) (layer F.Cu) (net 9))
 (segment (start 146.6 90.8) (end 146.6 91.8) (width 0.2) (layer F.Cu) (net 9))
 (segment (start 146.6 91.8) (end 146.7 91.9) (width 0.2) (layer F.Cu) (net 9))
 (segment (start 146.7 91.9) (end 146.9 91.9) (width 0.2) (layer F.Cu) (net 9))
 (segment (start 147 91.8) (end 147 90.8) (width 0.2) (layer F.Cu) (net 9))
 (segment (start 146.9 91.9) (end 147 91.8) (width 0.2) (layer F.Cu) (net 9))
 (segment (start 148.4 91.3) (end 147.8 91.3) (width 0.2) (layer F.Cu) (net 8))
 (segment (start 146.02805 90.55) (end 146.27805 90.3) (width 0.2) (layer F.Cu) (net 8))
 (segment (start 145 90.55) (end 146.02805 90.55) (width 0.2) (layer F.Cu) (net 8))
 (segment (start 146.27805 90.3) (end 148.4 90.3) (width 0.2) (layer F.Cu) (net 8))
 (segment (start 148.4 90.3) (end 148.6 90.5) (width 0.2) (layer F.Cu) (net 8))
 (segment (start 148.6 90.5) (end 148.6 91.1) (width 0.2) (layer F.Cu) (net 8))
 (segment (start 148.6 91.1) (end 148.4 91.3) (width 0.2) (layer F.Cu) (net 8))
 (segment (start 147.8 92.8) (end 150.8 92.8) (width 0.3) (layer F.Cu) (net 5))
 (segment (start 150.8 92.8) (end 151.6 93.6) (width 0.3) (layer F.Cu) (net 5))
 (segment (start 151.6 93.6) (end 153.1 93.6) (width 0.3) (layer F.Cu) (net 5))
 (via (at 154.1 94.5) (size 0.4) (drill 0.254) (layers F.Cu B.Cu) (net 5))
 (segment (start 153.1 93.6) (end 154 94.5) (width 0.3) (layer F.Cu) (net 5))
 (segment (start 154 94.5) (end 154.1 94.5) (width 0.3) (layer F.Cu) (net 5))
 (segment (start 159.143 94.5) (end 159.258 94.615) (width 0.3) (layer B.Cu) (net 5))
 (segment (start 154.1 94.5) (end 159.143 94.5) (width 0.3) (layer B.Cu) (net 5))
 (via (at 156.9 91.8) (size 0.4) (drill 0.254) (layers F.Cu B.Cu) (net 3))
 (segment (start 152.4 91.8) (end 156.9 91.8) (width 0.3) (layer F.Cu) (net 3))
 (segment (start 156.9 91.8) (end 156.9 91.7965) (width 0.3) (layer B.Cu) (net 3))
 (segment (start 159.1615 89.535) (end 159.258 89.535) (width 0.3) (layer B.Cu) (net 3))
 (segment (start 156.9 91.7965) (end 159.1615 89.535) (width 0.3) (layer B.Cu) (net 3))
 (segment (start 152.4 91.3) (end 156.1 91.3) (width 0.3) (layer F.Cu) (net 2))
 (via (at 156.2 91.2) (size 0.4) (drill 0.254) (layers F.Cu B.Cu) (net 2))
 (segment (start 156.1 91.3) (end 156.2 91.2) (width 0.3) (layer F.Cu) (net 2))
 (segment (start 156.2 91.2) (end 157.9 89.5) (width 0.3) (layer B.Cu) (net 2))
 (segment (start 157.9 88.353) (end 159.258 86.995) (width 0.3) (layer B.Cu) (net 2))
 (segment (start 157.9 89.5) (end 157.9 88.353) (width 0.3) (layer B.Cu) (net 2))
 (via (at 150.1 92.2) (size 0.4) (drill 0.254) (layers F.Cu B.Cu) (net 6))
 (segment (start 147.8 92.3) (end 150 92.3) (width 0.3) (layer F.Cu) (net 6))
 (segment (start 150 92.3) (end 150.1 92.2) (width 0.3) (layer F.Cu) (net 6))
 (segment (start 150.1 92.2) (end 151.9 90.4) (width 0.3) (layer B.Cu) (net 6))
 (segment (start 151.9 90.4) (end 155.9 90.4) (width 0.3) (layer B.Cu) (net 6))
 (segment (start 155.9 90.4) (end 157.2 89.1) (width 0.3) (layer B.Cu) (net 6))
 (segment (start 157.2 89.1) (end 157.2 88) (width 0.3) (layer B.Cu) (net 6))
 (segment (start 157.2 88) (end 157.9 87.3) (width 0.3) (layer B.Cu) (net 6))
 (segment (start 157.9 85.813) (end 159.258 84.455) (width 0.3) (layer B.Cu) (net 6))
 (segment (start 157.9 87.3) (end 157.9 85.813) (width 0.3) (layer B.Cu) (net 6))
 (segment (start 152.95 85.9) (end 152.95 84.4) (width 0.4) (layer F.Cu) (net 11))
 (segment (start 143.9 83.75) (end 145.4 83.75) (width 0.6) (layer F.Cu) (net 16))
 (segment (start 153.05 95.6) (end 153.05 97.2) (width 0.3) (layer F.Cu) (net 10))
 (segment (start 152.4 92.8) (end 153.3 92.8) (width 0.3) (layer F.Cu) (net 4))
 (segment (start 154.75 94.25) (end 154.75 95.6) (width 0.3) (layer F.Cu) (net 4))
 (segment (start 153.3 92.8) (end 154.75 94.25) (width 0.3) (layer F.Cu) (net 4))
 (segment (start 152.4 92.3) (end 151.101 92.3) (width 0.3) (layer F.Cu) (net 1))
 (segment (start 151.101 92.3) (end 150.864 92.063) (width 0.3) (layer F.Cu) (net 1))
 (segment (start 152.4 90.8) (end 150.881 90.8) (width 0.3) (layer F.Cu) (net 1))
 (segment (start 150.881 90.8) (end 150.864 90.817) (width 0.3) (layer F.Cu) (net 1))
 (segment (start 150.864 92.063) (end 150.864 90.817) (width 0.3) (layer F.Cu) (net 1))
 (segment (start 150.864 90.817) (end 150.864 89.027) (width 0.3) (layer F.Cu) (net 1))
 (segment (start 150.864 89.027) (end 150.864 88.436) (width 0.6) (layer F.Cu) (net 1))
 (segment (start 151.05 88.25) (end 151.05 87.45) (width 0.6) (layer F.Cu) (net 1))
 (segment (start 150.864 88.436) (end 151.05 88.25) (width 0.6) (layer F.Cu) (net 1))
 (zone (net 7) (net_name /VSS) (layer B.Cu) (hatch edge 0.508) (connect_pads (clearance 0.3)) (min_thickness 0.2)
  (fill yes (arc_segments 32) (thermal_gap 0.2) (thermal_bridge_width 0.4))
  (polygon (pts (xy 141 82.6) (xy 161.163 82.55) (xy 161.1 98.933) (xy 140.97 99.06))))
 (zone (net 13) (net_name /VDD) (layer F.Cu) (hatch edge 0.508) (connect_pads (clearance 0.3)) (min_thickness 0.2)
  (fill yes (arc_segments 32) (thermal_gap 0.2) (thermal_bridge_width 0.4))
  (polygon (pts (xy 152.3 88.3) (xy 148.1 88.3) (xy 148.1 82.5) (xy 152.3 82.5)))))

